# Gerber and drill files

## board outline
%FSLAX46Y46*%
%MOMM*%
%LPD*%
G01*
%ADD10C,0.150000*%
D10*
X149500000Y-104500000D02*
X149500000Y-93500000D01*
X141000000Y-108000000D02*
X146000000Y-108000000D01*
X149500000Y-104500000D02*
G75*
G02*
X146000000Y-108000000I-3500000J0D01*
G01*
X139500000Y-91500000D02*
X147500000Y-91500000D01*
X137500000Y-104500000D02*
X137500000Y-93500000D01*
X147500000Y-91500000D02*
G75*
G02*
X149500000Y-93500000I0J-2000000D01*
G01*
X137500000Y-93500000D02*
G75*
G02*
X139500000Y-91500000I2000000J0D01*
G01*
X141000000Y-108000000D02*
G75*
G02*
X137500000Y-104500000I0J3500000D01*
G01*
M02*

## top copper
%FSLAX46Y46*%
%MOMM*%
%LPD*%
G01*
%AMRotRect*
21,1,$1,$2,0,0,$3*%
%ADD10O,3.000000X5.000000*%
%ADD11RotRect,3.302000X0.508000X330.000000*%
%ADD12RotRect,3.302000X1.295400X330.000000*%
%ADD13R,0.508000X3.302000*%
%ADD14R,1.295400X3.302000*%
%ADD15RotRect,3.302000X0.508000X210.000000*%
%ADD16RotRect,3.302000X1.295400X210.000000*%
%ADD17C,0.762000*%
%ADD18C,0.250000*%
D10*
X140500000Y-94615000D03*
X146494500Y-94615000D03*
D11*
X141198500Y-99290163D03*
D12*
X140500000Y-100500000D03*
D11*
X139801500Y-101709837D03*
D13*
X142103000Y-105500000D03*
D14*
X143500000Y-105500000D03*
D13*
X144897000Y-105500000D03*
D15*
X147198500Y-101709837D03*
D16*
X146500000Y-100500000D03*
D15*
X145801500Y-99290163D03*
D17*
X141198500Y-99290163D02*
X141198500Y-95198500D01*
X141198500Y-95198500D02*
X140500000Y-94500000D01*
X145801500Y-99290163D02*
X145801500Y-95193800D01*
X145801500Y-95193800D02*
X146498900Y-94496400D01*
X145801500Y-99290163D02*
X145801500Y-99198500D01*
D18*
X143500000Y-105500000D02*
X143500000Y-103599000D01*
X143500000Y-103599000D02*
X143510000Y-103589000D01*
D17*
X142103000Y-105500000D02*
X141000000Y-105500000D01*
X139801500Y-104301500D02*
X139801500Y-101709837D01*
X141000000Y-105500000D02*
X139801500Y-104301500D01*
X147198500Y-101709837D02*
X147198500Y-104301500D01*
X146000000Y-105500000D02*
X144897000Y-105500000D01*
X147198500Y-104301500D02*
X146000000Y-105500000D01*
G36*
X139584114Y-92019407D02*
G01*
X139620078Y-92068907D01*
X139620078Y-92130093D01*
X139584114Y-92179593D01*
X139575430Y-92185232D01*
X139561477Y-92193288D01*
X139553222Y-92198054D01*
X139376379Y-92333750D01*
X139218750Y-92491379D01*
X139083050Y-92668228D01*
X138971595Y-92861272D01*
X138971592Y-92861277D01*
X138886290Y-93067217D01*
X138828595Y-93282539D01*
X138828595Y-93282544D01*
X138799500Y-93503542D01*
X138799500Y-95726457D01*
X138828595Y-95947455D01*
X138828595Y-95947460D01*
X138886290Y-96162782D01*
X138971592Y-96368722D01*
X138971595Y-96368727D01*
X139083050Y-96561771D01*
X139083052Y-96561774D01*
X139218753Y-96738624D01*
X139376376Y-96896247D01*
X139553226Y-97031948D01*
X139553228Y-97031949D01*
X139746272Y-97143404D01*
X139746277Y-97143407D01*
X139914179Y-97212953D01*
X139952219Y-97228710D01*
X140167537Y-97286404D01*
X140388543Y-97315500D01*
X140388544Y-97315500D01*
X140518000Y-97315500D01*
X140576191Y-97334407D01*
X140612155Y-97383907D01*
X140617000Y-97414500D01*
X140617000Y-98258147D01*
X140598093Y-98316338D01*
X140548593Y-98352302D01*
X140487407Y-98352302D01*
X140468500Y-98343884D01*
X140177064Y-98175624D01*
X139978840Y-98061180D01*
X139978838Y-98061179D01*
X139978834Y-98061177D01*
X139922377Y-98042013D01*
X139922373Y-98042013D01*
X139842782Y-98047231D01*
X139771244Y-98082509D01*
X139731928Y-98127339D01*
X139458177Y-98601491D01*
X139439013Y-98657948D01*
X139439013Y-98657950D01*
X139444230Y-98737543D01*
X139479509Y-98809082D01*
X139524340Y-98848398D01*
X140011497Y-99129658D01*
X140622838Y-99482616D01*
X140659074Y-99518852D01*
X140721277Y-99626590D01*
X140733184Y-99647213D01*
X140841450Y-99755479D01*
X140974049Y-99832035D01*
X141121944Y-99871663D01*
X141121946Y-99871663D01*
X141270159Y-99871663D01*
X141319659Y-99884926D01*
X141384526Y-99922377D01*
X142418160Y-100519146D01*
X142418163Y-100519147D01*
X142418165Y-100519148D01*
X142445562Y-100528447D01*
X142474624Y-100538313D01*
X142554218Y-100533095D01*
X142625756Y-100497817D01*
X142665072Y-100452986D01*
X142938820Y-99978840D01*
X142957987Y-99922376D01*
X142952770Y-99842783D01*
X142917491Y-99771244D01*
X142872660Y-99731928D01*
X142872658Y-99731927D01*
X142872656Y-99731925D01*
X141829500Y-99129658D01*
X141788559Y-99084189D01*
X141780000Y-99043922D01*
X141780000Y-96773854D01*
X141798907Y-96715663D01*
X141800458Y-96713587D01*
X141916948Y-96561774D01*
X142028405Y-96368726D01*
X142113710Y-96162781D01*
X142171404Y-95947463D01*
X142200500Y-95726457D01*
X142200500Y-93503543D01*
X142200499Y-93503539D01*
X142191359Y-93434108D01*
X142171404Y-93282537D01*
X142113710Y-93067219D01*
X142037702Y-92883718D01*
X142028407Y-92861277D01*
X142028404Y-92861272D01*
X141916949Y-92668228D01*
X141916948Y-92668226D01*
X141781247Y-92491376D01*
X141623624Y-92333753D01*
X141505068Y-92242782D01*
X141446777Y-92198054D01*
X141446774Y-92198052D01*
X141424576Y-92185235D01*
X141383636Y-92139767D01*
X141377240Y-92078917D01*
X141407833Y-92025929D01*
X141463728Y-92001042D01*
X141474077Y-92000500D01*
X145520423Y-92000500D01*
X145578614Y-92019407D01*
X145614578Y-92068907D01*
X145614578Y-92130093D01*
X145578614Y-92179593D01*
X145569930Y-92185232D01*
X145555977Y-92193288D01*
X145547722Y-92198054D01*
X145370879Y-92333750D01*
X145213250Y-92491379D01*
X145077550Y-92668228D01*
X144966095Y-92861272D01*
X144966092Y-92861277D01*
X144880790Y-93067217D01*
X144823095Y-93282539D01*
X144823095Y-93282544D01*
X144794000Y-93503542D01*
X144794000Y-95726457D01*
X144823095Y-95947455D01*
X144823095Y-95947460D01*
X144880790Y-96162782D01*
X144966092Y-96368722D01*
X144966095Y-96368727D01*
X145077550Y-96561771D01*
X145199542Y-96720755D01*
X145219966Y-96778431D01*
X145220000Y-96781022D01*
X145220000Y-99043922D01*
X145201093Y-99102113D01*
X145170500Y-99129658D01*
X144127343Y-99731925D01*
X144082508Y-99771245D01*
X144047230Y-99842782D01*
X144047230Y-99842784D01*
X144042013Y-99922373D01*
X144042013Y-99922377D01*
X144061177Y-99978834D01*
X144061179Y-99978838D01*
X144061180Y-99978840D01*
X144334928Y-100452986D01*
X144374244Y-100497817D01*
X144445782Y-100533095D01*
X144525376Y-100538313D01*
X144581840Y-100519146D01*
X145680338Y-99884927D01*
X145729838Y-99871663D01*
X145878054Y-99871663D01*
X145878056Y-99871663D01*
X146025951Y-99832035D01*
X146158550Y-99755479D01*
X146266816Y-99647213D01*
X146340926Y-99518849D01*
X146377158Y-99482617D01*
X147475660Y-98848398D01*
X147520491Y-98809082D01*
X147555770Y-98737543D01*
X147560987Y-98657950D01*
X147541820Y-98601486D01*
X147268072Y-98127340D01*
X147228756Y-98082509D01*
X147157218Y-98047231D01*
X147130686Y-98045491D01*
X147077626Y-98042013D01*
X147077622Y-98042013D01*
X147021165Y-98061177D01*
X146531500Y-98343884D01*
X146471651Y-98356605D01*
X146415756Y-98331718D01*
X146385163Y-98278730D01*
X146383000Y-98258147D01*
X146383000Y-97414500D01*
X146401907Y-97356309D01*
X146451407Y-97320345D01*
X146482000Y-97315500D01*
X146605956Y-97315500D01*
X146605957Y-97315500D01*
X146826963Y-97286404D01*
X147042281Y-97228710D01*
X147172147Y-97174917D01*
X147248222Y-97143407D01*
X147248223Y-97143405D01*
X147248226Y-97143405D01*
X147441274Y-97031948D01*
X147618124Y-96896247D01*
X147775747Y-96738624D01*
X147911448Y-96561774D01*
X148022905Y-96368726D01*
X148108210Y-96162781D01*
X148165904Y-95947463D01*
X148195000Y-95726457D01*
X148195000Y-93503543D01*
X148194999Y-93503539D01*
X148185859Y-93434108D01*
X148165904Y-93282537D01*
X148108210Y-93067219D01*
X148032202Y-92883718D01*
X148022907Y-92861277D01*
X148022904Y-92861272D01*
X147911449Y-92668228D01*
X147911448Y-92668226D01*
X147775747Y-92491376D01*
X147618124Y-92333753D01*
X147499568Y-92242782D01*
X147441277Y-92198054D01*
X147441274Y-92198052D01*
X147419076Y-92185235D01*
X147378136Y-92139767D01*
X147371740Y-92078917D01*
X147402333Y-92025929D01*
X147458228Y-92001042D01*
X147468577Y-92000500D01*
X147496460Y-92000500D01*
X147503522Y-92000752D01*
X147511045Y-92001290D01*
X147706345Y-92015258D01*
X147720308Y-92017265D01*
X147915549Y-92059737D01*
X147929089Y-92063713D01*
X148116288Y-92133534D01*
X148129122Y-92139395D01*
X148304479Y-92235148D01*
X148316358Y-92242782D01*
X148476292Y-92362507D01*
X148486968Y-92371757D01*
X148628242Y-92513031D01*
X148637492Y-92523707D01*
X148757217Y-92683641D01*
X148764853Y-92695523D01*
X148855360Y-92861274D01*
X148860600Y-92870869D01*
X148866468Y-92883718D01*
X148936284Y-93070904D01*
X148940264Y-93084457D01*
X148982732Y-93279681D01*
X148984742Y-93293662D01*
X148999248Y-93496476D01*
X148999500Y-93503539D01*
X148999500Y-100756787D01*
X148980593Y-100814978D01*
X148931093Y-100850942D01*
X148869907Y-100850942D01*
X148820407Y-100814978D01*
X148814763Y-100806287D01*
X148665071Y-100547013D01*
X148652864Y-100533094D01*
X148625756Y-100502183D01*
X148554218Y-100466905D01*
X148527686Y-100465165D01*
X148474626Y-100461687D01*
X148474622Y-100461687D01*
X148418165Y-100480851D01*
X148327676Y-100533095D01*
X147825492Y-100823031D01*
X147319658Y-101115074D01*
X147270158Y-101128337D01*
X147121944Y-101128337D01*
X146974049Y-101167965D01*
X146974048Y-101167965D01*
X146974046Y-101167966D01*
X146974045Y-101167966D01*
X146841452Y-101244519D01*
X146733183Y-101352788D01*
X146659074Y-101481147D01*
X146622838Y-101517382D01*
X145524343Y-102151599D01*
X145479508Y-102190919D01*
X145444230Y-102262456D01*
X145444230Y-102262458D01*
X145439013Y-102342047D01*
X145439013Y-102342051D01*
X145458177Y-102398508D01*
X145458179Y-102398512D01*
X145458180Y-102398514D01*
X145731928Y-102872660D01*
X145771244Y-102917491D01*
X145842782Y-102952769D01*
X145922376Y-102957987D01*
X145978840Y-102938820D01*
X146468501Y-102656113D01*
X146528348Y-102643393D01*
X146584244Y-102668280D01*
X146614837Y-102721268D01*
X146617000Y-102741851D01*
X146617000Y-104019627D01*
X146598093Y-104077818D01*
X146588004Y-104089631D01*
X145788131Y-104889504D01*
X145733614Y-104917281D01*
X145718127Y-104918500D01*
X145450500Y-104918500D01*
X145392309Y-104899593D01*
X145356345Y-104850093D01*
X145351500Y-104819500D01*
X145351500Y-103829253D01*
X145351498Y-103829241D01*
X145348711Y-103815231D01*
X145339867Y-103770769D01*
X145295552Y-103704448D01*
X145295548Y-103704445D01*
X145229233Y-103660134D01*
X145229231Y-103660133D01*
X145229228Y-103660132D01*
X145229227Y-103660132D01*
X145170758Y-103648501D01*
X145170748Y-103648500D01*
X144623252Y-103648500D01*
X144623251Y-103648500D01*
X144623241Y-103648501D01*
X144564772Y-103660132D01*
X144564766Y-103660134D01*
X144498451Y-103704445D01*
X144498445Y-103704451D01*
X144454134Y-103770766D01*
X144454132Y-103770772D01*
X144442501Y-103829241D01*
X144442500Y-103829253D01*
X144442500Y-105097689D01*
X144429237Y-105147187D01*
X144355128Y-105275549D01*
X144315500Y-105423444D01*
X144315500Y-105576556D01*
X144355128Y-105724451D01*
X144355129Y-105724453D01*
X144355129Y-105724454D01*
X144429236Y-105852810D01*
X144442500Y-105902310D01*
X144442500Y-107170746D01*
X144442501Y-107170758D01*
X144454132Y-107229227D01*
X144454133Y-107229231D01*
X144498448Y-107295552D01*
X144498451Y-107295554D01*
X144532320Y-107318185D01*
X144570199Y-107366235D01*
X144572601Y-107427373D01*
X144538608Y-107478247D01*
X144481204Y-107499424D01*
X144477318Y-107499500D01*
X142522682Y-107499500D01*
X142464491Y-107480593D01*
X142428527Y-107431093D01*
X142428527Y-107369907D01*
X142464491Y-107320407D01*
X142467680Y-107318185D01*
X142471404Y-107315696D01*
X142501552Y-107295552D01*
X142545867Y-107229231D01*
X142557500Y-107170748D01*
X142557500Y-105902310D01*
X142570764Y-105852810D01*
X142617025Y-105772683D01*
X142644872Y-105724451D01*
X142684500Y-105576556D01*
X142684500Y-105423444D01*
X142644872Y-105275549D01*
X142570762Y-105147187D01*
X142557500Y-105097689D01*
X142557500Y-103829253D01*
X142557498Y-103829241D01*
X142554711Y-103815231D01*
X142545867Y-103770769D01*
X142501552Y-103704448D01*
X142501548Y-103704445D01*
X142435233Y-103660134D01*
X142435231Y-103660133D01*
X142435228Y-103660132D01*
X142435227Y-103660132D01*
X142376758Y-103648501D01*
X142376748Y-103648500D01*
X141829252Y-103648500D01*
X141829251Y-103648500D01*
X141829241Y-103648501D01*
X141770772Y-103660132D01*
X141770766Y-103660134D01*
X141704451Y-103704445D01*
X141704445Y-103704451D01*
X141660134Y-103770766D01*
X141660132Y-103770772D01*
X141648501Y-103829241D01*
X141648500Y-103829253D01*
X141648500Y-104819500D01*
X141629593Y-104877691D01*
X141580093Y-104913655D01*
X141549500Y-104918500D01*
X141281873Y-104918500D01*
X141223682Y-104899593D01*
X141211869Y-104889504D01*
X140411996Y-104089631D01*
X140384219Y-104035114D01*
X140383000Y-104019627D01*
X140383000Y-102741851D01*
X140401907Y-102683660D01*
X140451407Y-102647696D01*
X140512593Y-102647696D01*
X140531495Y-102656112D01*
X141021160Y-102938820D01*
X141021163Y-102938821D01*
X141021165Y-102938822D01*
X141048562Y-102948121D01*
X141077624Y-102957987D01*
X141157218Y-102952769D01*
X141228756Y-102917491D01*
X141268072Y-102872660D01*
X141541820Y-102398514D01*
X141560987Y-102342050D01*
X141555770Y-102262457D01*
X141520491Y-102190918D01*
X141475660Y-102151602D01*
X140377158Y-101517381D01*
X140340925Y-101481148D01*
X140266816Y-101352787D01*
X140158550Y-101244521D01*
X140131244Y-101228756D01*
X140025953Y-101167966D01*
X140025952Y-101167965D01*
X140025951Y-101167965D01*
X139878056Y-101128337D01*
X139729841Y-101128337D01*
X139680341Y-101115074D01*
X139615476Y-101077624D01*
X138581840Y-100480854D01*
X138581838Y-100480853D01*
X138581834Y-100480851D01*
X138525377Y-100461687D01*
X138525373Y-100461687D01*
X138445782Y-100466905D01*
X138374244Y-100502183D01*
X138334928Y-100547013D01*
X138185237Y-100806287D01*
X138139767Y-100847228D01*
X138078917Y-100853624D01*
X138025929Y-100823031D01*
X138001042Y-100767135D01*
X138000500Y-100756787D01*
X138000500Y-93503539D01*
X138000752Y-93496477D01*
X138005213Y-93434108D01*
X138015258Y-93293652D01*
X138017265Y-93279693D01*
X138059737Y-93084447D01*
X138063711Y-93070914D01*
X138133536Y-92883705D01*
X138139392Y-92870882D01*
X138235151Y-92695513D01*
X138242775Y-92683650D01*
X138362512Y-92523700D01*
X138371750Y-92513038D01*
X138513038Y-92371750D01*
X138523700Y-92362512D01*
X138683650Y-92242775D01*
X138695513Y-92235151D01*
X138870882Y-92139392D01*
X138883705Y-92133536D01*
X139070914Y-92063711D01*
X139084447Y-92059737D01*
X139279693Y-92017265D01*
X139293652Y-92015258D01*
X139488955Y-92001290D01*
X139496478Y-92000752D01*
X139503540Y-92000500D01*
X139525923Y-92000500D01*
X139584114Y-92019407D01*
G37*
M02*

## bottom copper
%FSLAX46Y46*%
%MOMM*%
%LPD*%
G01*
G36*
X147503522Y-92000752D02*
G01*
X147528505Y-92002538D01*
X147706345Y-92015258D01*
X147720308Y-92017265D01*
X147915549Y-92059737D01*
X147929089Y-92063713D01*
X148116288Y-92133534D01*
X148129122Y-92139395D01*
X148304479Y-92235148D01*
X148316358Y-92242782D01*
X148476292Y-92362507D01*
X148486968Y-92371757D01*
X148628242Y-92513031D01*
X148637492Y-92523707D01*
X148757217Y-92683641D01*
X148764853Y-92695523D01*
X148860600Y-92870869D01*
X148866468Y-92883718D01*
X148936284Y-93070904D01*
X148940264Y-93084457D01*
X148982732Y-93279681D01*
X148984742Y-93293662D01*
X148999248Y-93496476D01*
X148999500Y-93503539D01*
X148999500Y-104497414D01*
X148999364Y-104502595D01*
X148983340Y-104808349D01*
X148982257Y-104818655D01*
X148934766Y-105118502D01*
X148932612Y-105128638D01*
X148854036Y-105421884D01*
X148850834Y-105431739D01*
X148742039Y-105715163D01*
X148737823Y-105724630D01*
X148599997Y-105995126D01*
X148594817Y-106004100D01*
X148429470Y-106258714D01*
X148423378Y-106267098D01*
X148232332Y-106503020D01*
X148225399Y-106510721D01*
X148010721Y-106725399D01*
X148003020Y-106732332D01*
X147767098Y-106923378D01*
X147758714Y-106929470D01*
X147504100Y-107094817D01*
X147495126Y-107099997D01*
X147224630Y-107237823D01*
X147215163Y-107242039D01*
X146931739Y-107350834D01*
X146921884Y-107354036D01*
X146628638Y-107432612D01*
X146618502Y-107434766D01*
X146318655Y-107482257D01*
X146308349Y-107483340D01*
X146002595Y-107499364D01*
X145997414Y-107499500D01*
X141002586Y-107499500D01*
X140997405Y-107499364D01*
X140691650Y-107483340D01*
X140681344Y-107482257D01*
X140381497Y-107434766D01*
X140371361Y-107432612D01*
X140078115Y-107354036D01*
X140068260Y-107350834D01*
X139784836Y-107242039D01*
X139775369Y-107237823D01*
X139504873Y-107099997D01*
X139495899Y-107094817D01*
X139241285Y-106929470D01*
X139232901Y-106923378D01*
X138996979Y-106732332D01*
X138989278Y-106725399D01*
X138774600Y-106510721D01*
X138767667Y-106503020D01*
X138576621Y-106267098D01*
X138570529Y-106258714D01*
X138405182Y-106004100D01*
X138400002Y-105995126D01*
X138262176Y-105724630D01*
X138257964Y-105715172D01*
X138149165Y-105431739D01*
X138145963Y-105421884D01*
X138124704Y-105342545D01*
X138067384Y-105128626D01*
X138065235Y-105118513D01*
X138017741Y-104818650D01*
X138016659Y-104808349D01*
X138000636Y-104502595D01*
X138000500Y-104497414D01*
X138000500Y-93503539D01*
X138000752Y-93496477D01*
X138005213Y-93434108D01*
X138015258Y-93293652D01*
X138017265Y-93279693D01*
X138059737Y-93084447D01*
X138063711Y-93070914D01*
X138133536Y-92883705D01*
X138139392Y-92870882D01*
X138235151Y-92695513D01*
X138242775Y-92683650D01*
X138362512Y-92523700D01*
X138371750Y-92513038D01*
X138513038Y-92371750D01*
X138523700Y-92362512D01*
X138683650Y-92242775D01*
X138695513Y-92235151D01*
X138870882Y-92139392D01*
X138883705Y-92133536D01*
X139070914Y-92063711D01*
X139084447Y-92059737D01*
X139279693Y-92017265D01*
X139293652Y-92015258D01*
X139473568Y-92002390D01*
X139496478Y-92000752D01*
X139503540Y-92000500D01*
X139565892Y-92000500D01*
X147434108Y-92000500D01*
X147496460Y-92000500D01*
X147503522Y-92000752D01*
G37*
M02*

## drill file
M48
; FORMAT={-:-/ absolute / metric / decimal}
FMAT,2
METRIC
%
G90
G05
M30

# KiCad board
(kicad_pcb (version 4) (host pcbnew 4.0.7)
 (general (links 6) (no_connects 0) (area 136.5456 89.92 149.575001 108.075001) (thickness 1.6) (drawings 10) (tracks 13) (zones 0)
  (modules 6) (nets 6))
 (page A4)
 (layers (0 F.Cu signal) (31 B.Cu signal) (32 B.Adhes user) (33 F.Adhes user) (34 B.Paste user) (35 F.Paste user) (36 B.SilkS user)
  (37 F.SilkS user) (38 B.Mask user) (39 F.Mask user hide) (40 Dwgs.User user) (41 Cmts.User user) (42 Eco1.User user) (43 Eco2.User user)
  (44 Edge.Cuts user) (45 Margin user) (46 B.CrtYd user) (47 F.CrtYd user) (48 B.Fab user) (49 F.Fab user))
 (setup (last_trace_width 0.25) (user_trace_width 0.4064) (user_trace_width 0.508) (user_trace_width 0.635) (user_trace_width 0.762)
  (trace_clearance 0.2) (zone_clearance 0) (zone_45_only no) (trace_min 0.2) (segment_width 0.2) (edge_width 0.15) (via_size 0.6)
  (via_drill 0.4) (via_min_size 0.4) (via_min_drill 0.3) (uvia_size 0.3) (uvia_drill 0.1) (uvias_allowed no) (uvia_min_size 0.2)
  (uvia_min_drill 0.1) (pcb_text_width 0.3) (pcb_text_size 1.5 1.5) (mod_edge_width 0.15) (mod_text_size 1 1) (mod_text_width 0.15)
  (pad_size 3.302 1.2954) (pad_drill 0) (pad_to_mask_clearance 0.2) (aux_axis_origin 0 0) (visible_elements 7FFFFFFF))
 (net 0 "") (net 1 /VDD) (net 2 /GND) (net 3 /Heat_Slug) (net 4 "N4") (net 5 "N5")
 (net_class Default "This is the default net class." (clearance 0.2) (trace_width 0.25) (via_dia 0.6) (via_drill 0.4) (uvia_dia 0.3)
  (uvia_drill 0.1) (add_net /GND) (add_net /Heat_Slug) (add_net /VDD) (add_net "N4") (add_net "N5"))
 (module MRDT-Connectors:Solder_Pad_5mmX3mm (layer F.Cu) (at 140.5 94.615)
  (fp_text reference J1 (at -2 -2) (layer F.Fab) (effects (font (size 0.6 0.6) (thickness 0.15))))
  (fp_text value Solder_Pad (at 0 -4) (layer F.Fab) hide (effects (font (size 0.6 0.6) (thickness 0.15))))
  (pad 1 smd oval (at 0 0) (size 3 5) (layers F.Cu F.Paste F.Mask) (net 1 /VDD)))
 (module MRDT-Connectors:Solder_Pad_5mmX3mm (layer F.Cu) (at 136.9956 93.6186)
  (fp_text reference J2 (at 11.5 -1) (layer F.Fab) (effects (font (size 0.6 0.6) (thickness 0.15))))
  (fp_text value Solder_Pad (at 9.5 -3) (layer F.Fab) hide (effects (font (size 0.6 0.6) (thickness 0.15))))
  (pad 1 smd oval (at 9.4989 0.9964) (size 3 5) (layers F.Cu F.Paste F.Mask) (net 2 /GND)))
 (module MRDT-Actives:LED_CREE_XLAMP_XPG (layer F.Cu) (at 140.5 100.5 240)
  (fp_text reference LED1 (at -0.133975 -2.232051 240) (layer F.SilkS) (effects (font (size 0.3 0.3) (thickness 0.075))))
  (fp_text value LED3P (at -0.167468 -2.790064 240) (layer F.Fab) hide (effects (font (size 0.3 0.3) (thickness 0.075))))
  (pad 1 smd rect (at -1.397 0 330) (size 3.302 0.508) (layers F.Cu F.Paste F.Mask) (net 1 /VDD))
  (pad 3 smd rect (at 0 0 330) (size 3.302 1.2954) (layers F.Cu F.Paste F.Mask) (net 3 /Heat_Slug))
  (pad 2 smd rect (at 1.397 0 330) (size 3.302 0.508) (layers F.Cu F.Paste F.Mask) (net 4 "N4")))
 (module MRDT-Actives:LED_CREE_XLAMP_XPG (layer F.Cu) (at 143.5 105.5)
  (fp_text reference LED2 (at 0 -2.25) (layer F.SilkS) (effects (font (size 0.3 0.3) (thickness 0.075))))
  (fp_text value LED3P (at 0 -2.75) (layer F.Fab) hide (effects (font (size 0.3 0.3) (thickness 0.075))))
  (pad 1 smd rect (at -1.397 0 90) (size 3.302 0.508) (layers F.Cu F.Paste F.Mask) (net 4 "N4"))
  (pad 3 smd rect (at 0 0 90) (size 3.302 1.2954) (layers F.Cu F.Paste F.Mask) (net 3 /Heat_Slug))
  (pad 2 smd rect (at 1.397 0 90) (size 3.302 0.508) (layers F.Cu F.Paste F.Mask) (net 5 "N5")))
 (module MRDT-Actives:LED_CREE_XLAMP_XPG (layer F.Cu) (at 146.5 100.5 120)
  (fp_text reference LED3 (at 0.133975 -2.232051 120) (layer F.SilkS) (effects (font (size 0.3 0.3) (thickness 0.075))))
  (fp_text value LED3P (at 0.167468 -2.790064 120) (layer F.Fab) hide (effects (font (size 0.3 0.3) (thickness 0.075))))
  (pad 1 smd rect (at -1.397 0 210) (size 3.302 0.508) (layers F.Cu F.Paste F.Mask) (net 5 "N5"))
  (pad 3 smd rect (at 0 0 210) (size 3.302 1.2954) (layers F.Cu F.Paste F.Mask) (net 3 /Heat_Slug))
  (pad 2 smd rect (at 1.397 0 210) (size 3.302 0.508) (layers F.Cu F.Paste F.Mask) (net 2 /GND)))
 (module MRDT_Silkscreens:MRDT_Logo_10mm (layer B.Cu) (at 142.9385 99.441 180)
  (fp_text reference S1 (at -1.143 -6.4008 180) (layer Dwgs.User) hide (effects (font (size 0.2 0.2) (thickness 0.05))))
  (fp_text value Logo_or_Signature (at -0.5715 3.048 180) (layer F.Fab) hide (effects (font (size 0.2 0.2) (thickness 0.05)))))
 (gr_line (start 149.5 104.5) (end 149.5 93.5) (angle 90) (layer Edge.Cuts) (width 0.15))
 (gr_line (start 141 108) (end 146 108) (angle 90) (layer Edge.Cuts) (width 0.15))
 (gr_arc (start 146 104.5) (end 149.5 104.5) (angle 90) (layer Edge.Cuts) (width 0.15))
 (gr_line (start 139.5 91.5) (end 147.5 91.5) (angle 90) (layer Edge.Cuts) (width 0.15))
 (gr_line (start 137.5 104.5) (end 137.5 93.5) (angle 90) (layer Edge.Cuts) (width 0.15))
 (gr_arc (start 147.5 93.5) (end 147.5 91.5) (angle 90) (layer Edge.Cuts) (width 0.15))
 (gr_arc (start 139.5 93.5) (end 137.5 93.5) (angle 90) (layer Edge.Cuts) (width 0.15))
 (gr_arc (start 141 104.5) (end 141 108) (angle 90) (layer Edge.Cuts) (width 0.15))
 (segment (start 141.1985 99.290163) (end 141.1985 95.1985) (width 0.762) (layer F.Cu) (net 1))
 (segment (start 141.1985 95.1985) (end 140.5 94.5) (width 0.762) (layer F.Cu) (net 1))
 (segment (start 145.8015 99.290163) (end 145.8015 95.1938) (width 0.762) (layer F.Cu) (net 2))
 (segment (start 145.8015 95.1938) (end 146.4989 94.4964) (width 0.762) (layer F.Cu) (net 2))
 (segment (start 145.8015 99.290163) (end 145.8015 99.1985) (width 0.762) (layer F.Cu) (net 2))
 (segment (start 143.5 105.5) (end 143.5 103.599) (width 0.25) (layer F.Cu) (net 3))
 (segment (start 143.5 103.599) (end 143.51 103.589) (width 0.25) (layer F.Cu) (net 3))
 (segment (start 142.103 105.5) (end 141 105.5) (width 0.762) (layer F.Cu) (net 4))
 (segment (start 139.8015 104.3015) (end 139.8015 101.709837) (width 0.762) (layer F.Cu) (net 4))
 (segment (start 141 105.5) (end 139.8015 104.3015) (width 0.762) (layer F.Cu) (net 4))
 (segment (start 147.1985 101.709837) (end 147.1985 104.3015) (width 0.762) (layer F.Cu) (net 5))
 (segment (start 146 105.5) (end 144.897 105.5) (width 0.762) (layer F.Cu) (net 5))
 (segment (start 147.1985 104.3015) (end 146 105.5) (width 0.762) (layer F.Cu) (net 5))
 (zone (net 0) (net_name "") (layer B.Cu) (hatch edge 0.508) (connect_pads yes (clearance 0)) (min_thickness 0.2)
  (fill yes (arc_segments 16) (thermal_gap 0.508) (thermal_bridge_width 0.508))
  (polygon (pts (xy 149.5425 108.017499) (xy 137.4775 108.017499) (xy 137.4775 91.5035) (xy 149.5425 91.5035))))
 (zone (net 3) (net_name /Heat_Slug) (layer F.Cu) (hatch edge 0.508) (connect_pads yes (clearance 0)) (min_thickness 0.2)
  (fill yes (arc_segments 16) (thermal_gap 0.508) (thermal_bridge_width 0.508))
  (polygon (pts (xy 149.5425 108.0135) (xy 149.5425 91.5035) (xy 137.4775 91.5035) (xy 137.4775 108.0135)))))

